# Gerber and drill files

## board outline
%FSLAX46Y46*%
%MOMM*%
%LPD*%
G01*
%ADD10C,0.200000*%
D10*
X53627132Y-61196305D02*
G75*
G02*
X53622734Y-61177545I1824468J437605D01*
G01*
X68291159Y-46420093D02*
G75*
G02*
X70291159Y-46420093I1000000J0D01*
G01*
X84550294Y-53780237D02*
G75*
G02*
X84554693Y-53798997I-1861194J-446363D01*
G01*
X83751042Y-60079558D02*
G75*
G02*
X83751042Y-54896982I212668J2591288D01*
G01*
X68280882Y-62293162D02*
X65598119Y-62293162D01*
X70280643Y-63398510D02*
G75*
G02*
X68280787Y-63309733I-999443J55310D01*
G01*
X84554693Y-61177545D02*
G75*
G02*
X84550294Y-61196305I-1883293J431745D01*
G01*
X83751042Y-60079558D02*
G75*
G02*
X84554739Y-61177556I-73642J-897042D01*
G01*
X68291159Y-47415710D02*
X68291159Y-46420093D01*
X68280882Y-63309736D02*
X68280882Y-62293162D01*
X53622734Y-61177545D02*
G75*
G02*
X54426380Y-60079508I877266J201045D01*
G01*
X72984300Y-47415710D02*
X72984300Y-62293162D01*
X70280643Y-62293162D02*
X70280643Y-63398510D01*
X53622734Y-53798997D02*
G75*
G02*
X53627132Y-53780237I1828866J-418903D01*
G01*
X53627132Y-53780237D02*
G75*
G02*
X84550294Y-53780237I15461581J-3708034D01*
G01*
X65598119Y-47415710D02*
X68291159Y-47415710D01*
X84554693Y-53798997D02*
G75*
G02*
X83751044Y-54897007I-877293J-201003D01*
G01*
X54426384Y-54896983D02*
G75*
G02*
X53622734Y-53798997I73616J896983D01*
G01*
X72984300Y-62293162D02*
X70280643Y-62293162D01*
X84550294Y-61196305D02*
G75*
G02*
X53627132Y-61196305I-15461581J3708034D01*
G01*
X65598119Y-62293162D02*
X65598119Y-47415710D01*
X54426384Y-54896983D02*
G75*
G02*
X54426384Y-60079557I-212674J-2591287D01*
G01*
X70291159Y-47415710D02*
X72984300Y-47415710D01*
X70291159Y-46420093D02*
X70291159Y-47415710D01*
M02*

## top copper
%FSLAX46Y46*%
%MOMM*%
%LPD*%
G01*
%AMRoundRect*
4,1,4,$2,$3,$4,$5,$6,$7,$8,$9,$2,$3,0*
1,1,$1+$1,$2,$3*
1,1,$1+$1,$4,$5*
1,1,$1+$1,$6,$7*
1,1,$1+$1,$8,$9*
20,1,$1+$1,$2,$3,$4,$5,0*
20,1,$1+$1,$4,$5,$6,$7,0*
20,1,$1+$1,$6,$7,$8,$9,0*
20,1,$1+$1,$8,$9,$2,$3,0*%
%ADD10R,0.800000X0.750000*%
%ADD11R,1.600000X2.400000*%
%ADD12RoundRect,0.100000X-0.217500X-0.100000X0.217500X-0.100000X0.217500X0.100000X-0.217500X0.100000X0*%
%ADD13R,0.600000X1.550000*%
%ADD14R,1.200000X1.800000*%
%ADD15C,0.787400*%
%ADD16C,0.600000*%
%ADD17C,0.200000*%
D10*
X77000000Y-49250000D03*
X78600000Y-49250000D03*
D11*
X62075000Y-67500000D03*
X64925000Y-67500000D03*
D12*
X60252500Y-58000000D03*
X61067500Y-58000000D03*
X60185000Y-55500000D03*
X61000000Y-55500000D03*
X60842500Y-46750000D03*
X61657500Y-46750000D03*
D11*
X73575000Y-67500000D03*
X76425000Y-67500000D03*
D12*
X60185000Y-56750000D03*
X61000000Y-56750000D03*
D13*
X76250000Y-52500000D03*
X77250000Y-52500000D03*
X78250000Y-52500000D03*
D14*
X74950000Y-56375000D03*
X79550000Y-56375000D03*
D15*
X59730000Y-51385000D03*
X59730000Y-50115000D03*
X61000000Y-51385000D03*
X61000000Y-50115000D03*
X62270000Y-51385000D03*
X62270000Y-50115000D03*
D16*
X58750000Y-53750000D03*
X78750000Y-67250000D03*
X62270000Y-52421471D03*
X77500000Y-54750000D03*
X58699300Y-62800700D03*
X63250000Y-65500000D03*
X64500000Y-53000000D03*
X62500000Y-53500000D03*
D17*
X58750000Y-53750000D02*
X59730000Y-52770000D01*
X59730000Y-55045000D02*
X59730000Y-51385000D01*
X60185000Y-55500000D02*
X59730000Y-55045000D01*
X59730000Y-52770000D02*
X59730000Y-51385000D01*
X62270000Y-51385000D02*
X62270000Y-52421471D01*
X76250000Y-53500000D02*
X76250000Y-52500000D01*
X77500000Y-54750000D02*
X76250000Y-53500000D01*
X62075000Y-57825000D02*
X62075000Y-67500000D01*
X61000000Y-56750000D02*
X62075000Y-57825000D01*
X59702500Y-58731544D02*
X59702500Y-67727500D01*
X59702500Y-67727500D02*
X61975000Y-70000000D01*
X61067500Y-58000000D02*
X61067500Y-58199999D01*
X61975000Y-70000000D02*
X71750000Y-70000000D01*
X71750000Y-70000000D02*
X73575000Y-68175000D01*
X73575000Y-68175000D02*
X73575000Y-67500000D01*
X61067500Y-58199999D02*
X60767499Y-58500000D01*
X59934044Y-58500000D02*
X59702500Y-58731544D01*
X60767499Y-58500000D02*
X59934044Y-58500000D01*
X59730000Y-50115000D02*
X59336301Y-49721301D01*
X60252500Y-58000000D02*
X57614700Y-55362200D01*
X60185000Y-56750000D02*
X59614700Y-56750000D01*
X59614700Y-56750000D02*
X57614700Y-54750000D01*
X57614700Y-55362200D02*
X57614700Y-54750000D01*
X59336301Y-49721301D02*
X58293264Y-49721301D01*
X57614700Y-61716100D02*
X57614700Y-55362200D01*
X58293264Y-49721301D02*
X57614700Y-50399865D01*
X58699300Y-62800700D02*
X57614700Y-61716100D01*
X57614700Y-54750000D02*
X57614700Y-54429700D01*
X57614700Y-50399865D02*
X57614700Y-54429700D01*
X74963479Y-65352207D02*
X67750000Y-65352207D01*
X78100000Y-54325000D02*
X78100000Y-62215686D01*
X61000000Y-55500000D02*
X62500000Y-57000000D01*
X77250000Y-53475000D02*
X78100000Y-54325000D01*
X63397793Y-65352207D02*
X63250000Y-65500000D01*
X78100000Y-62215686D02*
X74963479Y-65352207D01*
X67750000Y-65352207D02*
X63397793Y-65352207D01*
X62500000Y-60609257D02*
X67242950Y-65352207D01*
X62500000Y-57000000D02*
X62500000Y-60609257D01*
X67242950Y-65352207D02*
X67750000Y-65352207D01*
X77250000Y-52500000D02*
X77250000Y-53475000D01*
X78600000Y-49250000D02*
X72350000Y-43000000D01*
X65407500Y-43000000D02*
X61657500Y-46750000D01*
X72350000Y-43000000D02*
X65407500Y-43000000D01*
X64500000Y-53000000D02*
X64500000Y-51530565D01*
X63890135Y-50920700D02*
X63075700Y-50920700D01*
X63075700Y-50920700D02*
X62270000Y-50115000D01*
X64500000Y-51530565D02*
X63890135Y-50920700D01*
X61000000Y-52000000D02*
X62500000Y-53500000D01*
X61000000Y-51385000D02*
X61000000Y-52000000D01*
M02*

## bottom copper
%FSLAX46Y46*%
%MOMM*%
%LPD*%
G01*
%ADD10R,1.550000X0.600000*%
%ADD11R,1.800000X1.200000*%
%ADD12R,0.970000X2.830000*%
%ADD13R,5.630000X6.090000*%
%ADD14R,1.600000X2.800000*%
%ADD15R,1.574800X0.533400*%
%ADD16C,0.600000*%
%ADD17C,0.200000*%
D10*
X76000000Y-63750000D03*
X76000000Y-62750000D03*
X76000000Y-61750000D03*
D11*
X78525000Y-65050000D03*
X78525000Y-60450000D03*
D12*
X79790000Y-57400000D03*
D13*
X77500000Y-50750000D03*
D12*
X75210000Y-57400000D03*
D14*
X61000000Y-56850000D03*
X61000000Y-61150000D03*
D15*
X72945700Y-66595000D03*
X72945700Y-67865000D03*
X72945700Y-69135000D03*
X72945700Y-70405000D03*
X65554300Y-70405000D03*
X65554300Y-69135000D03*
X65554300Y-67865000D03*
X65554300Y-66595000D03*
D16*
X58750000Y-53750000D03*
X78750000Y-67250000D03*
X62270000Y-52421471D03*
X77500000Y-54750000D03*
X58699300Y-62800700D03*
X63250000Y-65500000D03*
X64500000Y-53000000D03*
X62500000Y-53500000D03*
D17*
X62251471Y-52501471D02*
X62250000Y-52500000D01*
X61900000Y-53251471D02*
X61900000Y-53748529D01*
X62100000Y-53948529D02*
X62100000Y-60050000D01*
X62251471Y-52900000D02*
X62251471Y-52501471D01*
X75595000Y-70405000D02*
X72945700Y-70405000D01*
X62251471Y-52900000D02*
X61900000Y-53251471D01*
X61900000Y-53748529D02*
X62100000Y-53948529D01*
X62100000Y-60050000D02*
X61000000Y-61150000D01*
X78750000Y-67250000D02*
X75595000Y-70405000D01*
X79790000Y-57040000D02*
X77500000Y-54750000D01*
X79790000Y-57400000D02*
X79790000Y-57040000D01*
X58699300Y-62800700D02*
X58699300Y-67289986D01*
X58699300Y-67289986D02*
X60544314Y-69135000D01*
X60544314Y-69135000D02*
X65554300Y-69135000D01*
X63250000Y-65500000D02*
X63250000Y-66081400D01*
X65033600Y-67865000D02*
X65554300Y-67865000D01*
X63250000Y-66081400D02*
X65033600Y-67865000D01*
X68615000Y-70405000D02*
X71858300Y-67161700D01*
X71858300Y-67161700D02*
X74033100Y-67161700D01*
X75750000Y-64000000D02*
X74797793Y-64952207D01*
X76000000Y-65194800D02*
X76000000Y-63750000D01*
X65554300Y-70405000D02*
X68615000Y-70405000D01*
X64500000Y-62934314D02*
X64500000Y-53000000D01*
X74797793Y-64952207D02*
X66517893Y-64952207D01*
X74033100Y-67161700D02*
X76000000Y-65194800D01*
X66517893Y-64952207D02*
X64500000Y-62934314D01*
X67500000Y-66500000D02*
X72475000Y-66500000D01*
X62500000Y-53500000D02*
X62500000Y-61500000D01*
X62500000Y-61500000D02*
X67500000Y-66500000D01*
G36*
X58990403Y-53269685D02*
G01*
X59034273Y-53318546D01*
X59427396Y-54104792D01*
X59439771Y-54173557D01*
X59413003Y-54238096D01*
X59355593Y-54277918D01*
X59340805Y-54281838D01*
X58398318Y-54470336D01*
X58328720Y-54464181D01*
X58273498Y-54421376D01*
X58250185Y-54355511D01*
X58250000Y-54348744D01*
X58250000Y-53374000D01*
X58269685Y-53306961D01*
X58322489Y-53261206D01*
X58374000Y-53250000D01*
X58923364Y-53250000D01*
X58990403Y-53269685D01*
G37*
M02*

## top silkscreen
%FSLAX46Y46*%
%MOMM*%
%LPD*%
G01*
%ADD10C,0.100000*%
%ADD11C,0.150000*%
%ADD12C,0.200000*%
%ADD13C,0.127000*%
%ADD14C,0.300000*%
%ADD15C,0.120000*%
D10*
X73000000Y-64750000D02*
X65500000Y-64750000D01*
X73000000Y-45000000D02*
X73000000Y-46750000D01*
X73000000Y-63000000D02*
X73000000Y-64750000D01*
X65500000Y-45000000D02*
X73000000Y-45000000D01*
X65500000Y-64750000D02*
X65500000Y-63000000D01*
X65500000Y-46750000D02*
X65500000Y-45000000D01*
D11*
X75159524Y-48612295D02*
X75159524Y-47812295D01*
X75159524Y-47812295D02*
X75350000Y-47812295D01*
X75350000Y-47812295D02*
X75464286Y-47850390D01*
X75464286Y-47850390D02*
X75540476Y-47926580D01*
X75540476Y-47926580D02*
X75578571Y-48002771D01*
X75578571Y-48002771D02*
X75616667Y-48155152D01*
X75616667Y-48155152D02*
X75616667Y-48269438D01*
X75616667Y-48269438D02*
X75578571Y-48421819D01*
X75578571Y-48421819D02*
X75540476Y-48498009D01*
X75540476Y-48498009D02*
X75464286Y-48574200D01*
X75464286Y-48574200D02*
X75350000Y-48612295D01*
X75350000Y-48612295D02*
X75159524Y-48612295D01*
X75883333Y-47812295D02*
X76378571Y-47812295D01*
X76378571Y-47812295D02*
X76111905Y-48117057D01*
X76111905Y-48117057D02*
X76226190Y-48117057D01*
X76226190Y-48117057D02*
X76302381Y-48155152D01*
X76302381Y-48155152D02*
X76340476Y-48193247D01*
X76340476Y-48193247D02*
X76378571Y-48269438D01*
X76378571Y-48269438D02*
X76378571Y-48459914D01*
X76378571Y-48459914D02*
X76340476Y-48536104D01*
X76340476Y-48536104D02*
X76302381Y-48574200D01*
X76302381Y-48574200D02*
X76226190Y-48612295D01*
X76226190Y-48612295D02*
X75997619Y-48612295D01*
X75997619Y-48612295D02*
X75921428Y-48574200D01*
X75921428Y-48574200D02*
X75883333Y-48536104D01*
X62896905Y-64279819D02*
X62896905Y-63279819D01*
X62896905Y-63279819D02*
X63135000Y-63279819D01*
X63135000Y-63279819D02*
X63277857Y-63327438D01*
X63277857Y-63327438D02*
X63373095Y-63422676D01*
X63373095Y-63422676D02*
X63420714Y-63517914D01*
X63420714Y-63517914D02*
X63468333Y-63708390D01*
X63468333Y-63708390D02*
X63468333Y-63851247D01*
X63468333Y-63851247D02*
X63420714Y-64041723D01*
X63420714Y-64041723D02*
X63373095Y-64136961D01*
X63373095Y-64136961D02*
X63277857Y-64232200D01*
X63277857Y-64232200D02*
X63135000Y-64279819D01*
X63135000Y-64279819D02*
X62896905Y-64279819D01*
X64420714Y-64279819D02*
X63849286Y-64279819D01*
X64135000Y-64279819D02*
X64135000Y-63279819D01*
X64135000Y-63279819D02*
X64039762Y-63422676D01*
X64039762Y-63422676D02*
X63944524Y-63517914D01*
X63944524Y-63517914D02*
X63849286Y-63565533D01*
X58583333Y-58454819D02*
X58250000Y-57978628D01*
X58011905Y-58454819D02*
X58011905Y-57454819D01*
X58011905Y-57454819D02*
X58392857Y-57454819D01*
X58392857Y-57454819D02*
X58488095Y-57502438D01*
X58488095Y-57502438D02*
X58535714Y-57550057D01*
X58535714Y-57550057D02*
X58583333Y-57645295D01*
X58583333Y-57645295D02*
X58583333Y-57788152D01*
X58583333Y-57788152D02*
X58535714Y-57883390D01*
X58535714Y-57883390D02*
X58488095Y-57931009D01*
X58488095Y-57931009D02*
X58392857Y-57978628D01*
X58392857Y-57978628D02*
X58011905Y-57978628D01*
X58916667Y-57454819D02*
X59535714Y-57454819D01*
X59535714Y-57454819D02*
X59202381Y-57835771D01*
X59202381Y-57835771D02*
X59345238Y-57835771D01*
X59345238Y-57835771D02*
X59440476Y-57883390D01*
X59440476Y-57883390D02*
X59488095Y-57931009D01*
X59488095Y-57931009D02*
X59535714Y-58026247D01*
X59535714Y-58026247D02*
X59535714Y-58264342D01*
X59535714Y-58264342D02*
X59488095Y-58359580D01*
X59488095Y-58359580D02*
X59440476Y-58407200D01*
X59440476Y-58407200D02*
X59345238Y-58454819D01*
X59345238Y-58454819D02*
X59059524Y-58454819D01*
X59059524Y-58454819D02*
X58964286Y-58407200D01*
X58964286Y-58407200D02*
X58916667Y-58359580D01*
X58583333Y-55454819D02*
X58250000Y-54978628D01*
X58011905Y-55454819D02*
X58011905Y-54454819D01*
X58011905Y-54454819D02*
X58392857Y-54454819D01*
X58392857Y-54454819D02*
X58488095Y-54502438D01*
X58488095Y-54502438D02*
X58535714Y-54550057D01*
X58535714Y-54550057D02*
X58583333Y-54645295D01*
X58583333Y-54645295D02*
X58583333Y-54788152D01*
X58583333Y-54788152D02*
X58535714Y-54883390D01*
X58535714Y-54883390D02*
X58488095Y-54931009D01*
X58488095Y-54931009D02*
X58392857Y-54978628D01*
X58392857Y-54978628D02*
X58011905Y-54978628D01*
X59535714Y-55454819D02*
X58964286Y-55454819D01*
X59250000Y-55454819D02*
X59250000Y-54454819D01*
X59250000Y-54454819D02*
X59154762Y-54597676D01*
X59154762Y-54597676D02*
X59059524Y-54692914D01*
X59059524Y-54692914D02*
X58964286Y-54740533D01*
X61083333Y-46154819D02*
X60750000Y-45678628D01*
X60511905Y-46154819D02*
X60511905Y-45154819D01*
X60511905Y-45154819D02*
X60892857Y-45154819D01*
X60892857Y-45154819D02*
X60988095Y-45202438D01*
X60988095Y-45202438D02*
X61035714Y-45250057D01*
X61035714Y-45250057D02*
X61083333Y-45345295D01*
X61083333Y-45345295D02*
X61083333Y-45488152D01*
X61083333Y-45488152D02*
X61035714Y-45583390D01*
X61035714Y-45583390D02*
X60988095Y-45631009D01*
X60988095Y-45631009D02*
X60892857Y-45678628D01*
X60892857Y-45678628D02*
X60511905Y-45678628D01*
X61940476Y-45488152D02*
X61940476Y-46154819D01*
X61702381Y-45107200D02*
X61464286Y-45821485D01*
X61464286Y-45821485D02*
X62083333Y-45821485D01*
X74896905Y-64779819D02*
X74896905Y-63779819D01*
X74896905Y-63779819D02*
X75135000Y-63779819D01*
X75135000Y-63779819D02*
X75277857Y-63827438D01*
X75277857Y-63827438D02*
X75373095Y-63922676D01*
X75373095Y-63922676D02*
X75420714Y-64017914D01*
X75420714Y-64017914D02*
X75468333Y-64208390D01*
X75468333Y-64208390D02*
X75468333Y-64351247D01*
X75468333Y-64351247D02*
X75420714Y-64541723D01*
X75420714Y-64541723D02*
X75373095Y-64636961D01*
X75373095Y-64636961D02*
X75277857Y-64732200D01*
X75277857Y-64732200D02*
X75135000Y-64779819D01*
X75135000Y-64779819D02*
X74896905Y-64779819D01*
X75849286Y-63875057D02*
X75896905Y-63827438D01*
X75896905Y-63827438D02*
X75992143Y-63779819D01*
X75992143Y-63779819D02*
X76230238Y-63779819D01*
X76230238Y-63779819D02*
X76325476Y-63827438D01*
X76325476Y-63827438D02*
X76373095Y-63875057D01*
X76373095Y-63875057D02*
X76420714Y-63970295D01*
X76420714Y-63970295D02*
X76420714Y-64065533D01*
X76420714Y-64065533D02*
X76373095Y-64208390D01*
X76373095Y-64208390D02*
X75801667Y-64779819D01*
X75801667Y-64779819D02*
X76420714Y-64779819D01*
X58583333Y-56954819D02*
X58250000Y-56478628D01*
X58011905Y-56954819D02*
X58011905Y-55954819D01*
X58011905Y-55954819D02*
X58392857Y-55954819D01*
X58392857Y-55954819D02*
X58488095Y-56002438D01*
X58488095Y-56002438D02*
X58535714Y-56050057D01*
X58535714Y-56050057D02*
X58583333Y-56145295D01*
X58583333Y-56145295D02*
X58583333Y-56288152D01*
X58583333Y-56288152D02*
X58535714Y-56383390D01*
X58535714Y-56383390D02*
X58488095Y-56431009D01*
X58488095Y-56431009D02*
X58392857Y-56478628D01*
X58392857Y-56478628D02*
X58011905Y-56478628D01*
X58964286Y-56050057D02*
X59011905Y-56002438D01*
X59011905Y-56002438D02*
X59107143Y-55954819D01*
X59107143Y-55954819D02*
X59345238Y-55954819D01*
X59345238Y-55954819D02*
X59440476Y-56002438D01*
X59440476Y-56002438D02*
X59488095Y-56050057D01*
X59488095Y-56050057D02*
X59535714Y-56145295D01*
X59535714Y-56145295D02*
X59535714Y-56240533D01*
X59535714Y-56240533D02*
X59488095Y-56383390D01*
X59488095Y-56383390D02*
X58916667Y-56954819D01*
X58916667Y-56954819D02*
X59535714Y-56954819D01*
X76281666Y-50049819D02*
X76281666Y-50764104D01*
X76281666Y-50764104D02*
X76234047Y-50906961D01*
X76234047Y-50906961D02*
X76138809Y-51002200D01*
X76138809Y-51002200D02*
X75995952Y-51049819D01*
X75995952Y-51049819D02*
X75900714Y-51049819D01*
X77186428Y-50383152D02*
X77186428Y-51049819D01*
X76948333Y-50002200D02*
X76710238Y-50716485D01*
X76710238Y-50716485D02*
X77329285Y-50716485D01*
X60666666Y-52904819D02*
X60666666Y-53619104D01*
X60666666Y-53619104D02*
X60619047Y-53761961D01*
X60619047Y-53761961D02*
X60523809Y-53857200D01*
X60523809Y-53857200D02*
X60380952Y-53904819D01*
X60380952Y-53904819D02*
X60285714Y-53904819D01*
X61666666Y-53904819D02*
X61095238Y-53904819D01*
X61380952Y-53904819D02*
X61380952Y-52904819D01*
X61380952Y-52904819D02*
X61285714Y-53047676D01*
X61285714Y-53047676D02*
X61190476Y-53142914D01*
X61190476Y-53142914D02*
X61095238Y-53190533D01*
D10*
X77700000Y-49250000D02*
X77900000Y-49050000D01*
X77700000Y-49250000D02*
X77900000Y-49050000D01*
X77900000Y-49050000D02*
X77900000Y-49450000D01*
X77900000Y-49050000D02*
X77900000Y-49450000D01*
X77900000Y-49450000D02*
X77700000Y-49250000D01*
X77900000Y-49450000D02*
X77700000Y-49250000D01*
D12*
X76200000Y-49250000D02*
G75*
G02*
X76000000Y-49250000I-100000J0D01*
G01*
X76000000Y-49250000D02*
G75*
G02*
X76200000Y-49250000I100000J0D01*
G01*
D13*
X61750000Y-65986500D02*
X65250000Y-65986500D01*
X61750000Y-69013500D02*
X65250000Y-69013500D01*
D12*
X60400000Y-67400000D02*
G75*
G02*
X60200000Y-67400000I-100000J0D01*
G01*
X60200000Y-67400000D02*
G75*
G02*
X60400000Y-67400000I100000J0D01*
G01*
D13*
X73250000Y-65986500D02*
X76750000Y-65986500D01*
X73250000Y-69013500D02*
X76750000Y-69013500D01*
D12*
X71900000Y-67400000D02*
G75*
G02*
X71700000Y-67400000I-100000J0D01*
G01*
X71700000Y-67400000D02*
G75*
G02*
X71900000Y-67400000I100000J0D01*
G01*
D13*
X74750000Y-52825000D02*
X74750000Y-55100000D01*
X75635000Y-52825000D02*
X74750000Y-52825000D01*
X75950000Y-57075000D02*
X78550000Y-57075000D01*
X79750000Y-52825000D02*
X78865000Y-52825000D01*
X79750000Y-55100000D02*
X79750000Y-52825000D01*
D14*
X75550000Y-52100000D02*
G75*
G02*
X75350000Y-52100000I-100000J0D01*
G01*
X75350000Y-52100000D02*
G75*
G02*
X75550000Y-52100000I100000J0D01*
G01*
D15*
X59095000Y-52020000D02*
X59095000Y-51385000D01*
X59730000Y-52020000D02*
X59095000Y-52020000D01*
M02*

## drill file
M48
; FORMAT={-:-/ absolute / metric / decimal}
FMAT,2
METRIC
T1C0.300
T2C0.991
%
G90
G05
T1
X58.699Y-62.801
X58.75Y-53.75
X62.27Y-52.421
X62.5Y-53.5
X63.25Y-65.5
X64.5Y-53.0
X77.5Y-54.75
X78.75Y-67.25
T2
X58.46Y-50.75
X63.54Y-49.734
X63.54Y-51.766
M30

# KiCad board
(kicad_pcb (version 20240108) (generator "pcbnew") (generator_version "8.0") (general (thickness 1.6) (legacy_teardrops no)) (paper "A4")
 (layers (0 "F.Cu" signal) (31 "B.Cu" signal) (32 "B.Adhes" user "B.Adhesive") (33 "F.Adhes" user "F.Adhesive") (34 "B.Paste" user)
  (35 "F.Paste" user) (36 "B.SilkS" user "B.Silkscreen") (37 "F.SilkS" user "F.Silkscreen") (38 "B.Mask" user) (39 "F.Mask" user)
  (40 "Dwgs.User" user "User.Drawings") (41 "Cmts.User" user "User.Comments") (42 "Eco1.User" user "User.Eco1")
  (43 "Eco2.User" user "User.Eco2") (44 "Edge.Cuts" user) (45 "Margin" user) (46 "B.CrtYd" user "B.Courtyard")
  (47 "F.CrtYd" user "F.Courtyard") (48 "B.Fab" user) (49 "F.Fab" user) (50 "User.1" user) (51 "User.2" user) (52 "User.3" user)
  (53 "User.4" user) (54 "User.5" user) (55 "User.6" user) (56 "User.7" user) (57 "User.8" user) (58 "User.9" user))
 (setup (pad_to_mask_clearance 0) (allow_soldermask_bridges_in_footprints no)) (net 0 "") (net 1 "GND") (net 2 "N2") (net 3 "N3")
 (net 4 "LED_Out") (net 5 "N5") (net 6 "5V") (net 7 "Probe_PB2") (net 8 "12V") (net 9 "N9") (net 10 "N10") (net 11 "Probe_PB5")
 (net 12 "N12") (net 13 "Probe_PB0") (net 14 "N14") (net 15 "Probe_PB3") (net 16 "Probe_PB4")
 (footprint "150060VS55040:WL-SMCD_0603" (layer "F.Cu") (at 77.8 49.25)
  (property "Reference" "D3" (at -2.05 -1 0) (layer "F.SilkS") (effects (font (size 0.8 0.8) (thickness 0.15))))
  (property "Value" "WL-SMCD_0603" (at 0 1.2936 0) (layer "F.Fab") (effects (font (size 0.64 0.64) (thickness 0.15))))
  (fp_line (start -0.1 0) (end 0.1 -0.2) (stroke (width 0.1) (type solid)) (layer "F.SilkS"))
  (fp_line (start -0.1 0) (end 0.1 -0.2) (stroke (width 0.1) (type solid)) (layer "F.SilkS"))
  (fp_line (start 0.1 -0.2) (end 0.1 0.2) (stroke (width 0.1) (type solid)) (layer "F.SilkS"))
  (fp_line (start 0.1 -0.2) (end 0.1 0.2) (stroke (width 0.1) (type solid)) (layer "F.SilkS"))
  (fp_line (start 0.1 0.2) (end -0.1 0) (stroke (width 0.1) (type solid)) (layer "F.SilkS"))
  (fp_line (start 0.1 0.2) (end -0.1 0) (stroke (width 0.1) (type solid)) (layer "F.SilkS"))
  (fp_circle (center -1.7 0) (end -1.6 0) (stroke (width 0.2) (type solid)) (fill none) (layer "F.SilkS"))
  (pad "1" smd rect (at -0.8 0) (size 0.8 0.75) (layers "F.Cu" "F.Paste" "F.Mask") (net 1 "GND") (solder_mask_margin 0.102))
  (pad "2" smd rect (at 0.8 0) (size 0.8 0.75) (layers "F.Cu" "F.Paste" "F.Mask") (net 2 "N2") (solder_mask_margin 0.102)))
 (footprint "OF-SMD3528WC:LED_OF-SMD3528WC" (layer "F.Cu") (at 63.5 67.5)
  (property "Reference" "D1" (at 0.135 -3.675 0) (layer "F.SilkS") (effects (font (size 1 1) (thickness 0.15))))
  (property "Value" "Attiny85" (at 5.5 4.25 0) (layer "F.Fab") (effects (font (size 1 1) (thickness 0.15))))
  (fp_line (start -1.75 -1.5135) (end 1.75 -1.5135) (stroke (width 0.127) (type solid)) (layer "F.SilkS"))
  (fp_line (start -1.75 1.5135) (end 1.75 1.5135) (stroke (width 0.127) (type solid)) (layer "F.SilkS"))
  (fp_circle (center -3.2 -0.1) (end -3.1 -0.1) (stroke (width 0.2) (type solid)) (fill none) (layer "F.SilkS"))
  (pad "1" smd rect (at -1.425 0) (size 1.6 2.4) (layers "F.Cu" "F.Paste" "F.Mask") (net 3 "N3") (solder_mask_margin 0.102))
  (pad "2" smd rect (at 1.425 0) (size 1.6 2.4) (layers "F.Cu" "F.Paste" "F.Mask") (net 1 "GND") (solder_mask_margin 0.102)))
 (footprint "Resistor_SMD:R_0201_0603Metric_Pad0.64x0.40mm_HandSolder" (layer "F.Cu") (at 60.66 58)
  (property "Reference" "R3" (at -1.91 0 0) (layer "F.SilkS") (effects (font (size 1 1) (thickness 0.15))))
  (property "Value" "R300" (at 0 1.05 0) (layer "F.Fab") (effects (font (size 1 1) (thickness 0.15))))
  (pad "" smd roundrect (at -0.4325 0) (size 0.458 0.36) (layers "F.Paste") (roundrect_rratio 0.25))
  (pad "" smd roundrect (at 0.4325 0) (size 0.458 0.36) (layers "F.Paste") (roundrect_rratio 0.25))
  (pad "1" smd roundrect (at -0.4075 0) (size 0.635 0.4) (layers "F.Cu" "F.Mask") (roundrect_rratio 0.25) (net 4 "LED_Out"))
  (pad "2" smd roundrect (at 0.4075 0) (size 0.635 0.4) (layers "F.Cu" "F.Mask") (roundrect_rratio 0.25) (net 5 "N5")))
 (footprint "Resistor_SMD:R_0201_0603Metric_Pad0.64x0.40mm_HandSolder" (layer "F.Cu") (at 60.5925 55.5)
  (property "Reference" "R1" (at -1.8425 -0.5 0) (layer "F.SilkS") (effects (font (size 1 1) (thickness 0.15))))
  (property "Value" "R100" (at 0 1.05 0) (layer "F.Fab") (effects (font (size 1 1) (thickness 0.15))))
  (pad "" smd roundrect (at -0.4325 0) (size 0.458 0.36) (layers "F.Paste") (roundrect_rratio 0.25))
  (pad "" smd roundrect (at 0.4325 0) (size 0.458 0.36) (layers "F.Paste") (roundrect_rratio 0.25))
  (pad "1" smd roundrect (at -0.4075 0) (size 0.635 0.4) (layers "F.Cu" "F.Mask") (roundrect_rratio 0.25) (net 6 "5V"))
  (pad "2" smd roundrect (at 0.4075 0) (size 0.635 0.4) (layers "F.Cu" "F.Mask") (roundrect_rratio 0.25) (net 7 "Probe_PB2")))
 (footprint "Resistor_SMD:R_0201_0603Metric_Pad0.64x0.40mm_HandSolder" (layer "F.Cu") (at 61.25 46.75)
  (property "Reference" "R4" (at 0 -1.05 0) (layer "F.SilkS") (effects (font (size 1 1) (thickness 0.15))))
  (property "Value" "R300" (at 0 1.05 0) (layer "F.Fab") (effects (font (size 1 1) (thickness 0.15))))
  (pad "" smd roundrect (at -0.4325 0) (size 0.458 0.36) (layers "F.Paste") (roundrect_rratio 0.25))
  (pad "" smd roundrect (at 0.4325 0) (size 0.458 0.36) (layers "F.Paste") (roundrect_rratio 0.25))
  (pad "1" smd roundrect (at -0.4075 0) (size 0.635 0.4) (layers "F.Cu" "F.Mask") (roundrect_rratio 0.25) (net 6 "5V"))
  (pad "2" smd roundrect (at 0.4075 0) (size 0.635 0.4) (layers "F.Cu" "F.Mask") (roundrect_rratio 0.25) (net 2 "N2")))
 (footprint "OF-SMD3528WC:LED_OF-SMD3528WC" (layer "F.Cu") (at 75 67.5)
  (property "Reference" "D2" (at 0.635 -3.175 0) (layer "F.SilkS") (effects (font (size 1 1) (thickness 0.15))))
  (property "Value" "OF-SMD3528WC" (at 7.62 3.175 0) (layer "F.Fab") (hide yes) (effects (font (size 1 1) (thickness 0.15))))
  (fp_line (start -1.75 -1.5135) (end 1.75 -1.5135) (stroke (width 0.127) (type solid)) (layer "F.SilkS"))
  (fp_line (start -1.75 1.5135) (end 1.75 1.5135) (stroke (width 0.127) (type solid)) (layer "F.SilkS"))
  (fp_circle (center -3.2 -0.1) (end -3.1 -0.1) (stroke (width 0.2) (type solid)) (fill none) (layer "F.SilkS"))
  (pad "1" smd rect (at -1.425 0) (size 1.6 2.4) (layers "F.Cu" "F.Paste" "F.Mask") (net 5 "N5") (solder_mask_margin 0.102))
  (pad "2" smd rect (at 1.425 0) (size 1.6 2.4) (layers "F.Cu" "F.Paste" "F.Mask") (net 1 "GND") (solder_mask_margin 0.102)))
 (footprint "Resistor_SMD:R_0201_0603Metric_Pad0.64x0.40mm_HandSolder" (layer "F.Cu") (at 60.5925 56.75)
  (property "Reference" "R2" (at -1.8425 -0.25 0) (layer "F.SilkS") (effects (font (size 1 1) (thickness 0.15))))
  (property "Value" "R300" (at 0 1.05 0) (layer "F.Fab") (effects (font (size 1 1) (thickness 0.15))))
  (pad "" smd roundrect (at -0.4325 0) (size 0.458 0.36) (layers "F.Paste") (roundrect_rratio 0.25))
  (pad "" smd roundrect (at 0.4325 0) (size 0.458 0.36) (layers "F.Paste") (roundrect_rratio 0.25))
  (pad "1" smd roundrect (at -0.4075 0) (size 0.635 0.4) (layers "F.Cu" "F.Mask") (roundrect_rratio 0.25) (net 4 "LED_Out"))
  (pad "2" smd roundrect (at 0.4075 0) (size 0.635 0.4) (layers "F.Cu" "F.Mask") (roundrect_rratio 0.25) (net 3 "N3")))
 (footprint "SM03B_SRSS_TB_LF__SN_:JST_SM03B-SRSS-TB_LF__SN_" (layer "F.Cu") (at 77.25 52.5)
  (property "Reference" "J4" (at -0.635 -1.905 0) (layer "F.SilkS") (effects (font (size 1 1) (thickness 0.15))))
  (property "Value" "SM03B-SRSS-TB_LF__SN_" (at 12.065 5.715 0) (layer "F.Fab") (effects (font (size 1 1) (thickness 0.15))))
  (fp_line (start -2.5 0.325) (end -2.5 2.6) (stroke (width 0.127) (type solid)) (layer "F.SilkS"))
  (fp_line (start -1.615 0.325) (end -2.5 0.325) (stroke (width 0.127) (type solid)) (layer "F.SilkS"))
  (fp_line (start -1.3 4.575) (end 1.3 4.575) (stroke (width 0.127) (type solid)) (layer "F.SilkS"))
  (fp_line (start 2.5 0.325) (end 1.615 0.325) (stroke (width 0.127) (type solid)) (layer "F.SilkS"))
  (fp_line (start 2.5 2.6) (end 2.5 0.325) (stroke (width 0.127) (type solid)) (layer "F.SilkS"))
  (fp_circle (center -1.8 -0.4) (end -1.7 -0.4) (stroke (width 0.3) (type solid)) (fill none) (layer "F.SilkS"))
  (pad "1" smd rect (at -1 0) (size 0.6 1.55) (layers "F.Cu" "F.Paste" "F.Mask") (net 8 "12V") (solder_mask_margin 0.102))
  (pad "2" smd rect (at 0 0) (size 0.6 1.55) (layers "F.Cu" "F.Paste" "F.Mask") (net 7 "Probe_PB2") (solder_mask_margin 0.102))
  (pad "3" smd rect (at 1 0) (size 0.6 1.55) (layers "F.Cu" "F.Paste" "F.Mask") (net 1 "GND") (solder_mask_margin 0.102))
  (pad "S1" smd rect (at -2.3 3.875) (size 1.2 1.8) (layers "F.Cu" "F.Paste" "F.Mask") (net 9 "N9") (solder_mask_margin 0.102))
  (pad "S2" smd rect (at 2.3 3.875) (size 1.2 1.8) (layers "F.Cu" "F.Paste" "F.Mask") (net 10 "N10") (solder_mask_margin 0.102)))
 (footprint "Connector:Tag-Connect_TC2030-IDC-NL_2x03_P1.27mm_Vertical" (layer "F.Cu") (at 61 50.75)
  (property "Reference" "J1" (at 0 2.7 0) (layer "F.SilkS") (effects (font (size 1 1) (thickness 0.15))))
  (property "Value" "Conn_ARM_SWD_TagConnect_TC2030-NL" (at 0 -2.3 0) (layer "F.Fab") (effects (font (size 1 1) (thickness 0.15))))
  (fp_line (start -1.905 1.27) (end -1.905 0.635) (stroke (width 0.12) (type solid)) (layer "F.SilkS"))
  (fp_line (start -1.27 1.27) (end -1.905 1.27) (stroke (width 0.12) (type solid)) (layer "F.SilkS"))
  (pad "" np_thru_hole circle (at -2.54 0) (size 0.9906 0.9906) (drill 0.9906) (layers "*.Cu" "*.Mask"))
  (pad "" np_thru_hole circle (at 2.54 -1.016) (size 0.9906 0.9906) (drill 0.9906) (layers "*.Cu" "*.Mask"))
  (pad "" np_thru_hole circle (at 2.54 1.016) (size 0.9906 0.9906) (drill 0.9906) (layers "*.Cu" "*.Mask"))
  (pad "1" connect circle (at -1.27 0.635) (size 0.7874 0.7874) (layers "F.Cu" "F.Mask") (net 6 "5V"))
  (pad "2" connect circle (at -1.27 -0.635) (size 0.7874 0.7874) (layers "F.Cu" "F.Mask") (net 4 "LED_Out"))
  (pad "3" connect circle (at 0 0.635) (size 0.7874 0.7874) (layers "F.Cu" "F.Mask") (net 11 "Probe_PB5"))
  (pad "4" connect circle (at 0 -0.635) (size 0.7874 0.7874) (layers "F.Cu" "F.Mask") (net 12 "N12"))
  (pad "5" connect circle (at 1.27 0.635) (size 0.7874 0.7874) (layers "F.Cu" "F.Mask") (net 1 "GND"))
  (pad "6" connect circle (at 1.27 -0.635) (size 0.7874 0.7874) (layers "F.Cu" "F.Mask") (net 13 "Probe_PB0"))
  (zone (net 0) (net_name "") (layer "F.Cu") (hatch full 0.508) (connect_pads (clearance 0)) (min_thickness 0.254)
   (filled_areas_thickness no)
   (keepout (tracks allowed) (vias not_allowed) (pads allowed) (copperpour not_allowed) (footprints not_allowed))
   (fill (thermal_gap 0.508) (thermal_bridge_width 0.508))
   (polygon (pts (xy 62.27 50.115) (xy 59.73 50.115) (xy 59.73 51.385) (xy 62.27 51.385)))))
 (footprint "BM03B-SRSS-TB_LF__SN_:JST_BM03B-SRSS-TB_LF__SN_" (layer "B.Cu") (at 78.525 62.75 90)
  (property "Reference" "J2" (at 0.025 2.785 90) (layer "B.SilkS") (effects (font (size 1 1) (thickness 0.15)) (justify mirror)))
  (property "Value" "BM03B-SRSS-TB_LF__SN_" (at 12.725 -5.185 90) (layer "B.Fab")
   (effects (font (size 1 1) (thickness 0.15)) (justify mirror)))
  (pad "1" smd rect (at -1 -2.525 90) (size 0.6 1.55) (layers "B.Cu" "B.Paste" "B.Mask") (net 13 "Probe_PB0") (solder_mask_margin 0.102))
  (pad "2" smd rect (at 0 -2.525 90) (size 0.6 1.55) (layers "B.Cu" "B.Paste" "B.Mask") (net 6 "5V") (solder_mask_margin 0.102))
  (pad "3" smd rect (at 1 -2.525 90) (size 0.6 1.55) (layers "B.Cu" "B.Paste" "B.Mask") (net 1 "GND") (solder_mask_margin 0.102))
  (pad "S1" smd rect (at -2.3 0 90) (size 1.2 1.8) (layers "B.Cu" "B.Paste" "B.Mask") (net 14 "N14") (solder_mask_margin 0.102))
  (pad "S2" smd rect (at 2.3 0 90) (size 1.2 1.8) (layers "B.Cu" "B.Paste" "B.Mask") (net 14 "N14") (solder_mask_margin 0.102)))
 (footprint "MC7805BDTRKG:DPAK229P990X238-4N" (layer "B.Cu") (at 77.5 53.26 180)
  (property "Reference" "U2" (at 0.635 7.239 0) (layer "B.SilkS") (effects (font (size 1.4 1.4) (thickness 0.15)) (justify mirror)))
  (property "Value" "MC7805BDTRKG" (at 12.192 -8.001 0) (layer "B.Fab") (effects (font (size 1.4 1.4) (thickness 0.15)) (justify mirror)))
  (pad "1" smd rect (at -2.29 -4.14 180) (size 0.97 2.83) (layers "B.Cu" "B.Paste" "B.Mask") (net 8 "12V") (solder_mask_margin 0.102))
  (pad "2" smd rect (at 0 2.51 180) (size 5.63 6.09) (layers "B.Cu" "B.Mask") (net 1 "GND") (solder_mask_margin 0.102))
  (pad "3" smd rect (at 2.29 -4.14 180) (size 0.97 2.83) (layers "B.Cu" "B.Paste" "B.Mask") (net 6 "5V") (solder_mask_margin 0.102)))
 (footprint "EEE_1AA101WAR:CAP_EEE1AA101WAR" (layer "B.Cu") (at 61 59 -90)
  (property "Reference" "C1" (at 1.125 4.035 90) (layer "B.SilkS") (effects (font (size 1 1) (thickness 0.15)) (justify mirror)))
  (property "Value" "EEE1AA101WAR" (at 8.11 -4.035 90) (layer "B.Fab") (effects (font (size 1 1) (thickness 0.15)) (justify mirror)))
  (pad "1" smd rect (at -2.15 0 270) (size 2.8 1.6) (layers "B.Cu" "B.Paste" "B.Mask") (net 6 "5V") (solder_mask_margin 0.102))
  (pad "2" smd rect (at 2.15 0 270) (size 2.8 1.6) (layers "B.Cu" "B.Paste" "B.Mask") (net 1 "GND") (solder_mask_margin 0.102)))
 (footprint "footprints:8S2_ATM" (layer "B.Cu") (at 69.25 68.5 180)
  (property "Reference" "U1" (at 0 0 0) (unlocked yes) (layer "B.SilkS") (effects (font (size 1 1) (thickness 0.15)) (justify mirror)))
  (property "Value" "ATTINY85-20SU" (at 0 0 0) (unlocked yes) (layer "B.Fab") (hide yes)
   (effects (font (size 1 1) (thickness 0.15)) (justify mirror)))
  (pad "1" smd rect (at -3.6957 1.905 180) (size 1.5748 0.5334) (layers "B.Cu" "B.Paste" "B.Mask") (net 11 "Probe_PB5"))
  (pad "2" smd rect (at -3.6957 0.635 180) (size 1.5748 0.5334) (layers "B.Cu" "B.Paste" "B.Mask") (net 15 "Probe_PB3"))
  (pad "3" smd rect (at -3.6957 -0.635 180) (size 1.5748 0.5334) (layers "B.Cu" "B.Paste" "B.Mask") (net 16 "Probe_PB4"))
  (pad "4" smd rect (at -3.6957 -1.905 180) (size 1.5748 0.5334) (layers "B.Cu" "B.Paste" "B.Mask") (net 1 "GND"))
  (pad "5" smd rect (at 3.6957 -1.905 180) (size 1.5748 0.5334) (layers "B.Cu" "B.Paste" "B.Mask") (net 13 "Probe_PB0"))
  (pad "6" smd rect (at 3.6957 -0.635 180) (size 1.5748 0.5334) (layers "B.Cu" "B.Paste" "B.Mask") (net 4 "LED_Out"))
  (pad "7" smd rect (at 3.6957 0.635 180) (size 1.5748 0.5334) (layers "B.Cu" "B.Paste" "B.Mask") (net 7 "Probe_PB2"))
  (pad "8" smd rect (at 3.6957 1.905 180) (size 1.5748 0.5334) (layers "B.Cu" "B.Paste" "B.Mask") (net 6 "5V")))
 (gr_line (start 73 64.75) (end 65.5 64.75) (stroke (width 0.1) (type default)) (layer "F.SilkS"))
 (gr_line (start 73 45) (end 73 46.75) (stroke (width 0.1) (type default)) (layer "F.SilkS"))
 (gr_line (start 73 63) (end 73 64.75) (stroke (width 0.1) (type default)) (layer "F.SilkS"))
 (gr_line (start 65.5 45) (end 73 45) (stroke (width 0.1) (type default)) (layer "F.SilkS"))
 (gr_line (start 65.5 64.75) (end 65.5 63) (stroke (width 0.1) (type default)) (layer "F.SilkS"))
 (gr_line (start 65.5 46.75) (end 65.5 45) (stroke (width 0.1) (type default)) (layer "F.SilkS"))
 (gr_arc (start 53.627132 61.196305) (mid 53.624909 61.186931) (end 53.622734 61.177545) (stroke (width 0.2) (type default))
  (layer "Edge.Cuts"))
 (gr_arc (start 68.291159 46.420093) (mid 69.291159 45.420093) (end 70.291159 46.420093) (stroke (width 0.2) (type default))
  (layer "Edge.Cuts"))
 (gr_arc (start 84.550294 53.780237) (mid 84.552517 53.789611) (end 84.554693 53.798997) (stroke (width 0.2) (type default))
  (layer "Edge.Cuts"))
 (gr_arc (start 83.751042 60.079558) (mid 81.363712 57.488273) (end 83.751042 54.896983) (stroke (width 0.2) (type default))
  (layer "Edge.Cuts"))
 (gr_line (start 68.280882 62.293162) (end 65.598119 62.293162) (stroke (width 0.2) (type default)) (layer "Edge.Cuts"))
 (gr_arc (start 70.280643 63.39851) (mid 69.236859 64.343094) (end 68.280882 63.309736) (stroke (width 0.2) (type default))
  (layer "Edge.Cuts"))
 (gr_arc (start 84.554693 61.177545) (mid 84.552517 61.18693) (end 84.550294 61.196305) (stroke (width 0.2) (type default))
  (layer "Edge.Cuts"))
 (gr_arc (start 83.751042 60.079558) (mid 84.403671 60.444979) (end 84.554693 61.177545) (stroke (width 0.2) (type default))
  (layer "Edge.Cuts"))
 (gr_line (start 68.291159 47.41571) (end 68.291159 46.420093) (stroke (width 0.2) (type default)) (layer "Edge.Cuts"))
 (gr_line (start 68.280882 63.309736) (end 68.280882 62.293162) (stroke (width 0.2) (type default)) (layer "Edge.Cuts"))
 (gr_arc (start 53.622734 61.177545) (mid 53.773752 60.444979) (end 54.426384 60.079558) (stroke (width 0.2) (type default))
  (layer "Edge.Cuts"))
 (gr_line (start 72.9843 47.41571) (end 72.9843 62.293162) (stroke (width 0.2) (type default)) (layer "Edge.Cuts"))
 (gr_line (start 70.280643 62.293162) (end 70.280643 63.39851) (stroke (width 0.2) (type default)) (layer "Edge.Cuts"))
 (gr_arc (start 53.622734 53.798997) (mid 53.624909 53.789611) (end 53.627132 53.780237) (stroke (width 0.2) (type default))
  (layer "Edge.Cuts"))
 (gr_arc (start 53.627132 53.780237) (mid 69.088713 41.588271) (end 84.550294 53.780237) (stroke (width 0.2) (type default))
  (layer "Edge.Cuts"))
 (gr_line (start 65.598119 47.41571) (end 68.291159 47.41571) (stroke (width 0.2) (type default)) (layer "Edge.Cuts"))
 (gr_arc (start 84.554693 53.798997) (mid 84.403673 54.53157) (end 83.751042 54.896983) (stroke (width 0.2) (type default))
  (layer "Edge.Cuts"))
 (gr_arc (start 54.426384 54.896983) (mid 53.773751 54.531564) (end 53.622734 53.798997) (stroke (width 0.2) (type default))
  (layer "Edge.Cuts"))
 (gr_line (start 72.9843 62.293162) (end 70.280643 62.293162) (stroke (width 0.2) (type default)) (layer "Edge.Cuts"))
 (gr_arc (start 84.550294 61.196305) (mid 69.088713 73.388271) (end 53.627132 61.196305) (stroke (width 0.2) (type default))
  (layer "Edge.Cuts"))
 (gr_line (start 65.598119 62.293162) (end 65.598119 47.41571) (stroke (width 0.2) (type default)) (layer "Edge.Cuts"))
 (gr_arc (start 54.426384 54.896983) (mid 56.813713 57.488271) (end 54.426384 60.079558) (stroke (width 0.2) (type default))
  (layer "Edge.Cuts"))
 (gr_line (start 70.291159 47.41571) (end 72.9843 47.41571) (stroke (width 0.2) (type default)) (layer "Edge.Cuts"))
 (gr_line (start 70.291159 46.420093) (end 70.291159 47.41571) (stroke (width 0.2) (type default)) (layer "Edge.Cuts"))
 (segment (start 58.75 53.75) (end 59.73 52.77) (width 0.2) (layer "F.Cu") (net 6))
 (segment (start 59.73 55.045) (end 59.73 51.385) (width 0.2) (layer "F.Cu") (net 6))
 (segment (start 60.185 55.5) (end 59.73 55.045) (width 0.2) (layer "F.Cu") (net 6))
 (segment (start 59.73 52.77) (end 59.73 51.385) (width 0.2) (layer "F.Cu") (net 6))
 (via (at 58.75 53.75) (size 0.6) (drill 0.3) (layers "F.Cu" "B.Cu") (free yes) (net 6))
 (segment (start 62.27 51.385) (end 62.27 52.421471) (width 0.2) (layer "F.Cu") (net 1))
 (via (at 78.75 67.25) (size 0.6) (drill 0.3) (layers "F.Cu" "B.Cu") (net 1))
 (via (at 62.27 52.421471) (size 0.6) (drill 0.3) (layers "F.Cu" "B.Cu") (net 1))
 (segment (start 62.251471 52.501471) (end 62.25 52.5) (width 0.2) (layer "B.Cu") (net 1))
 (segment (start 61.9 53.251471) (end 61.9 53.748529) (width 0.2) (layer "B.Cu") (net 1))
 (segment (start 62.1 53.948529) (end 62.1 60.05) (width 0.2) (layer "B.Cu") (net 1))
 (segment (start 62.251471 52.9) (end 62.251471 52.501471) (width 0.2) (layer "B.Cu") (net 1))
 (segment (start 75.595 70.405) (end 72.9457 70.405) (width 0.2) (layer "B.Cu") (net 1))
 (segment (start 62.251471 52.9) (end 61.9 53.251471) (width 0.2) (layer "B.Cu") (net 1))
 (segment (start 61.9 53.748529) (end 62.1 53.948529) (width 0.2) (layer "B.Cu") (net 1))
 (segment (start 62.1 60.05) (end 61 61.15) (width 0.2) (layer "B.Cu") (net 1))
 (segment (start 78.75 67.25) (end 75.595 70.405) (width 0.2) (layer "B.Cu") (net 1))
 (segment (start 76.25 53.5) (end 76.25 52.5) (width 0.2) (layer "F.Cu") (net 8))
 (segment (start 77.5 54.75) (end 76.25 53.5) (width 0.2) (layer "F.Cu") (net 8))
 (via (at 77.5 54.75) (size 0.6) (drill 0.3) (layers "F.Cu" "B.Cu") (free yes) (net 8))
 (segment (start 79.79 57.04) (end 77.5 54.75) (width 0.2) (layer "B.Cu") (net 8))
 (segment (start 79.79 57.4) (end 79.79 57.04) (width 0.2) (layer "B.Cu") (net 8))
 (segment (start 62.075 57.825) (end 62.075 67.5) (width 0.2) (layer "F.Cu") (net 3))
 (segment (start 61 56.75) (end 62.075 57.825) (width 0.2) (layer "F.Cu") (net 3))
 (segment (start 59.7025 58.731544) (end 59.7025 67.7275) (width 0.2) (layer "F.Cu") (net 5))
 (segment (start 59.7025 67.7275) (end 61.975 70) (width 0.2) (layer "F.Cu") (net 5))
 (segment (start 61.0675 58) (end 61.0675 58.199999) (width 0.2) (layer "F.Cu") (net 5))
 (segment (start 61.975 70) (end 71.75 70) (width 0.2) (layer "F.Cu") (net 5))
 (segment (start 71.75 70) (end 73.575 68.175) (width 0.2) (layer "F.Cu") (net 5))
 (segment (start 73.575 68.175) (end 73.575 67.5) (width 0.2) (layer "F.Cu") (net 5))
 (segment (start 61.0675 58.199999) (end 60.767499 58.5) (width 0.2) (layer "F.Cu") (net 5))
 (segment (start 59.934044 58.5) (end 59.7025 58.731544) (width 0.2) (layer "F.Cu") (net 5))
 (segment (start 60.767499 58.5) (end 59.934044 58.5) (width 0.2) (layer "F.Cu") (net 5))
 (segment (start 59.73 50.115) (end 59.336301 49.721301) (width 0.2) (layer "F.Cu") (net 4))
 (segment (start 60.2525 58) (end 57.6147 55.3622) (width 0.2) (layer "F.Cu") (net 4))
 (segment (start 60.185 56.75) (end 59.6147 56.75) (width 0.2) (layer "F.Cu") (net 4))
 (segment (start 59.6147 56.75) (end 57.6147 54.75) (width 0.2) (layer "F.Cu") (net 4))
 (segment (start 57.6147 55.3622) (end 57.6147 54.75) (width 0.2) (layer "F.Cu") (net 4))
 (segment (start 59.336301 49.721301) (end 58.293264 49.721301) (width 0.2) (layer "F.Cu") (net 4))
 (segment (start 57.6147 61.7161) (end 57.6147 55.3622) (width 0.2) (layer "F.Cu") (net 4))
 (segment (start 58.293264 49.721301) (end 57.6147 50.399865) (width 0.2) (layer "F.Cu") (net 4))
 (segment (start 58.6993 62.8007) (end 57.6147 61.7161) (width 0.2) (layer "F.Cu") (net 4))
 (segment (start 57.6147 54.75) (end 57.6147 54.4297) (width 0.2) (layer "F.Cu") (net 4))
 (segment (start 57.6147 50.399865) (end 57.6147 54.4297) (width 0.2) (layer "F.Cu") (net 4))
 (via (at 58.6993 62.8007) (size 0.6) (drill 0.3) (layers "F.Cu" "B.Cu") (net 4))
 (segment (start 58.6993 62.8007) (end 58.6993 67.289986) (width 0.2) (layer "B.Cu") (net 4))
 (segment (start 58.6993 67.289986) (end 60.544314 69.135) (width 0.2) (layer "B.Cu") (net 4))
 (segment (start 60.544314 69.135) (end 65.5543 69.135) (width 0.2) (layer "B.Cu") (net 4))
 (segment (start 74.963479 65.352207) (end 67.75 65.352207) (width 0.2) (layer "F.Cu") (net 7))
 (segment (start 78.1 54.325) (end 78.1 62.215686) (width 0.2) (layer "F.Cu") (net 7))
 (segment (start 61 55.5) (end 62.5 57) (width 0.2) (layer "F.Cu") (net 7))
 (segment (start 77.25 53.475) (end 78.1 54.325) (width 0.2) (layer "F.Cu") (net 7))
 (segment (start 63.397793 65.352207) (end 63.25 65.5) (width 0.2) (layer "F.Cu") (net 7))
 (segment (start 78.1 62.215686) (end 74.963479 65.352207) (width 0.2) (layer "F.Cu") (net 7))
 (segment (start 67.75 65.352207) (end 63.397793 65.352207) (width 0.2) (layer "F.Cu") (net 7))
 (segment (start 62.5 60.609257) (end 67.24295 65.352207) (width 0.2) (layer "F.Cu") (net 7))
 (segment (start 62.5 57) (end 62.5 60.609257) (width 0.2) (layer "F.Cu") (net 7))
 (segment (start 67.24295 65.352207) (end 67.75 65.352207) (width 0.2) (layer "F.Cu") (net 7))
 (segment (start 77.25 52.5) (end 77.25 53.475) (width 0.2) (layer "F.Cu") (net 7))
 (via (at 63.25 65.5) (size 0.6) (drill 0.3) (layers "F.Cu" "B.Cu") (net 7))
 (segment (start 63.25 65.5) (end 63.25 66.0814) (width 0.2) (layer "B.Cu") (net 7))
 (segment (start 65.0336 67.865) (end 65.5543 67.865) (width 0.2) (layer "B.Cu") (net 7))
 (segment (start 63.25 66.0814) (end 65.0336 67.865) (width 0.2) (layer "B.Cu") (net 7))
 (segment (start 78.6 49.25) (end 72.35 43) (width 0.2) (layer "F.Cu") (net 2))
 (segment (start 65.4075 43) (end 61.6575 46.75) (width 0.2) (layer "F.Cu") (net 2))
 (segment (start 72.35 43) (end 65.4075 43) (width 0.2) (layer "F.Cu") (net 2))
 (segment (start 64.5 53) (end 64.5 51.530565) (width 0.2) (layer "F.Cu") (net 13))
 (segment (start 63.890135 50.9207) (end 63.0757 50.9207) (width 0.2) (layer "F.Cu") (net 13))
 (segment (start 63.0757 50.9207) (end 62.27 50.115) (width 0.2) (layer "F.Cu") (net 13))
 (segment (start 64.5 51.530565) (end 63.890135 50.9207) (width 0.2) (layer "F.Cu") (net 13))
 (via (at 64.5 53) (size 0.6) (drill 0.3) (layers "F.Cu" "B.Cu") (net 13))
 (segment (start 68.615 70.405) (end 71.8583 67.1617) (width 0.2) (layer "B.Cu") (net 13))
 (segment (start 71.8583 67.1617) (end 74.0331 67.1617) (width 0.2) (layer "B.Cu") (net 13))
 (segment (start 75.75 64) (end 74.797793 64.952207) (width 0.2) (layer "B.Cu") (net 13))
 (segment (start 76 65.1948) (end 76 63.75) (width 0.2) (layer "B.Cu") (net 13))
 (segment (start 65.5543 70.405) (end 68.615 70.405) (width 0.2) (layer "B.Cu") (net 13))
 (segment (start 64.5 62.934314) (end 64.5 53) (width 0.2) (layer "B.Cu") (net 13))
 (segment (start 74.797793 64.952207) (end 66.517893 64.952207) (width 0.2) (layer "B.Cu") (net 13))
 (segment (start 74.0331 67.1617) (end 76 65.1948) (width 0.2) (layer "B.Cu") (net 13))
 (segment (start 66.517893 64.952207) (end 64.5 62.934314) (width 0.2) (layer "B.Cu") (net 13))
 (segment (start 61 52) (end 62.5 53.5) (width 0.2) (layer "F.Cu") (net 11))
 (segment (start 61 51.385) (end 61 52) (width 0.2) (layer "F.Cu") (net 11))
 (via (at 62.5 53.5) (size 0.6) (drill 0.3) (layers "F.Cu" "B.Cu") (free yes) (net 11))
 (segment (start 67.5 66.5) (end 72.475 66.5) (width 0.2) (layer "B.Cu") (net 11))
 (segment (start 62.5 53.5) (end 62.5 61.5) (width 0.2) (layer "B.Cu") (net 11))
 (segment (start 62.5 61.5) (end 67.5 66.5) (width 0.2) (layer "B.Cu") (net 11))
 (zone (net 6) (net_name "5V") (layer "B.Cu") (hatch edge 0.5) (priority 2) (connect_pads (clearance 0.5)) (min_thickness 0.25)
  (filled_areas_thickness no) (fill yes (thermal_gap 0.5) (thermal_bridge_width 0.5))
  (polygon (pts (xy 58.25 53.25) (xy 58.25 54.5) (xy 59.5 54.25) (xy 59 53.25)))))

